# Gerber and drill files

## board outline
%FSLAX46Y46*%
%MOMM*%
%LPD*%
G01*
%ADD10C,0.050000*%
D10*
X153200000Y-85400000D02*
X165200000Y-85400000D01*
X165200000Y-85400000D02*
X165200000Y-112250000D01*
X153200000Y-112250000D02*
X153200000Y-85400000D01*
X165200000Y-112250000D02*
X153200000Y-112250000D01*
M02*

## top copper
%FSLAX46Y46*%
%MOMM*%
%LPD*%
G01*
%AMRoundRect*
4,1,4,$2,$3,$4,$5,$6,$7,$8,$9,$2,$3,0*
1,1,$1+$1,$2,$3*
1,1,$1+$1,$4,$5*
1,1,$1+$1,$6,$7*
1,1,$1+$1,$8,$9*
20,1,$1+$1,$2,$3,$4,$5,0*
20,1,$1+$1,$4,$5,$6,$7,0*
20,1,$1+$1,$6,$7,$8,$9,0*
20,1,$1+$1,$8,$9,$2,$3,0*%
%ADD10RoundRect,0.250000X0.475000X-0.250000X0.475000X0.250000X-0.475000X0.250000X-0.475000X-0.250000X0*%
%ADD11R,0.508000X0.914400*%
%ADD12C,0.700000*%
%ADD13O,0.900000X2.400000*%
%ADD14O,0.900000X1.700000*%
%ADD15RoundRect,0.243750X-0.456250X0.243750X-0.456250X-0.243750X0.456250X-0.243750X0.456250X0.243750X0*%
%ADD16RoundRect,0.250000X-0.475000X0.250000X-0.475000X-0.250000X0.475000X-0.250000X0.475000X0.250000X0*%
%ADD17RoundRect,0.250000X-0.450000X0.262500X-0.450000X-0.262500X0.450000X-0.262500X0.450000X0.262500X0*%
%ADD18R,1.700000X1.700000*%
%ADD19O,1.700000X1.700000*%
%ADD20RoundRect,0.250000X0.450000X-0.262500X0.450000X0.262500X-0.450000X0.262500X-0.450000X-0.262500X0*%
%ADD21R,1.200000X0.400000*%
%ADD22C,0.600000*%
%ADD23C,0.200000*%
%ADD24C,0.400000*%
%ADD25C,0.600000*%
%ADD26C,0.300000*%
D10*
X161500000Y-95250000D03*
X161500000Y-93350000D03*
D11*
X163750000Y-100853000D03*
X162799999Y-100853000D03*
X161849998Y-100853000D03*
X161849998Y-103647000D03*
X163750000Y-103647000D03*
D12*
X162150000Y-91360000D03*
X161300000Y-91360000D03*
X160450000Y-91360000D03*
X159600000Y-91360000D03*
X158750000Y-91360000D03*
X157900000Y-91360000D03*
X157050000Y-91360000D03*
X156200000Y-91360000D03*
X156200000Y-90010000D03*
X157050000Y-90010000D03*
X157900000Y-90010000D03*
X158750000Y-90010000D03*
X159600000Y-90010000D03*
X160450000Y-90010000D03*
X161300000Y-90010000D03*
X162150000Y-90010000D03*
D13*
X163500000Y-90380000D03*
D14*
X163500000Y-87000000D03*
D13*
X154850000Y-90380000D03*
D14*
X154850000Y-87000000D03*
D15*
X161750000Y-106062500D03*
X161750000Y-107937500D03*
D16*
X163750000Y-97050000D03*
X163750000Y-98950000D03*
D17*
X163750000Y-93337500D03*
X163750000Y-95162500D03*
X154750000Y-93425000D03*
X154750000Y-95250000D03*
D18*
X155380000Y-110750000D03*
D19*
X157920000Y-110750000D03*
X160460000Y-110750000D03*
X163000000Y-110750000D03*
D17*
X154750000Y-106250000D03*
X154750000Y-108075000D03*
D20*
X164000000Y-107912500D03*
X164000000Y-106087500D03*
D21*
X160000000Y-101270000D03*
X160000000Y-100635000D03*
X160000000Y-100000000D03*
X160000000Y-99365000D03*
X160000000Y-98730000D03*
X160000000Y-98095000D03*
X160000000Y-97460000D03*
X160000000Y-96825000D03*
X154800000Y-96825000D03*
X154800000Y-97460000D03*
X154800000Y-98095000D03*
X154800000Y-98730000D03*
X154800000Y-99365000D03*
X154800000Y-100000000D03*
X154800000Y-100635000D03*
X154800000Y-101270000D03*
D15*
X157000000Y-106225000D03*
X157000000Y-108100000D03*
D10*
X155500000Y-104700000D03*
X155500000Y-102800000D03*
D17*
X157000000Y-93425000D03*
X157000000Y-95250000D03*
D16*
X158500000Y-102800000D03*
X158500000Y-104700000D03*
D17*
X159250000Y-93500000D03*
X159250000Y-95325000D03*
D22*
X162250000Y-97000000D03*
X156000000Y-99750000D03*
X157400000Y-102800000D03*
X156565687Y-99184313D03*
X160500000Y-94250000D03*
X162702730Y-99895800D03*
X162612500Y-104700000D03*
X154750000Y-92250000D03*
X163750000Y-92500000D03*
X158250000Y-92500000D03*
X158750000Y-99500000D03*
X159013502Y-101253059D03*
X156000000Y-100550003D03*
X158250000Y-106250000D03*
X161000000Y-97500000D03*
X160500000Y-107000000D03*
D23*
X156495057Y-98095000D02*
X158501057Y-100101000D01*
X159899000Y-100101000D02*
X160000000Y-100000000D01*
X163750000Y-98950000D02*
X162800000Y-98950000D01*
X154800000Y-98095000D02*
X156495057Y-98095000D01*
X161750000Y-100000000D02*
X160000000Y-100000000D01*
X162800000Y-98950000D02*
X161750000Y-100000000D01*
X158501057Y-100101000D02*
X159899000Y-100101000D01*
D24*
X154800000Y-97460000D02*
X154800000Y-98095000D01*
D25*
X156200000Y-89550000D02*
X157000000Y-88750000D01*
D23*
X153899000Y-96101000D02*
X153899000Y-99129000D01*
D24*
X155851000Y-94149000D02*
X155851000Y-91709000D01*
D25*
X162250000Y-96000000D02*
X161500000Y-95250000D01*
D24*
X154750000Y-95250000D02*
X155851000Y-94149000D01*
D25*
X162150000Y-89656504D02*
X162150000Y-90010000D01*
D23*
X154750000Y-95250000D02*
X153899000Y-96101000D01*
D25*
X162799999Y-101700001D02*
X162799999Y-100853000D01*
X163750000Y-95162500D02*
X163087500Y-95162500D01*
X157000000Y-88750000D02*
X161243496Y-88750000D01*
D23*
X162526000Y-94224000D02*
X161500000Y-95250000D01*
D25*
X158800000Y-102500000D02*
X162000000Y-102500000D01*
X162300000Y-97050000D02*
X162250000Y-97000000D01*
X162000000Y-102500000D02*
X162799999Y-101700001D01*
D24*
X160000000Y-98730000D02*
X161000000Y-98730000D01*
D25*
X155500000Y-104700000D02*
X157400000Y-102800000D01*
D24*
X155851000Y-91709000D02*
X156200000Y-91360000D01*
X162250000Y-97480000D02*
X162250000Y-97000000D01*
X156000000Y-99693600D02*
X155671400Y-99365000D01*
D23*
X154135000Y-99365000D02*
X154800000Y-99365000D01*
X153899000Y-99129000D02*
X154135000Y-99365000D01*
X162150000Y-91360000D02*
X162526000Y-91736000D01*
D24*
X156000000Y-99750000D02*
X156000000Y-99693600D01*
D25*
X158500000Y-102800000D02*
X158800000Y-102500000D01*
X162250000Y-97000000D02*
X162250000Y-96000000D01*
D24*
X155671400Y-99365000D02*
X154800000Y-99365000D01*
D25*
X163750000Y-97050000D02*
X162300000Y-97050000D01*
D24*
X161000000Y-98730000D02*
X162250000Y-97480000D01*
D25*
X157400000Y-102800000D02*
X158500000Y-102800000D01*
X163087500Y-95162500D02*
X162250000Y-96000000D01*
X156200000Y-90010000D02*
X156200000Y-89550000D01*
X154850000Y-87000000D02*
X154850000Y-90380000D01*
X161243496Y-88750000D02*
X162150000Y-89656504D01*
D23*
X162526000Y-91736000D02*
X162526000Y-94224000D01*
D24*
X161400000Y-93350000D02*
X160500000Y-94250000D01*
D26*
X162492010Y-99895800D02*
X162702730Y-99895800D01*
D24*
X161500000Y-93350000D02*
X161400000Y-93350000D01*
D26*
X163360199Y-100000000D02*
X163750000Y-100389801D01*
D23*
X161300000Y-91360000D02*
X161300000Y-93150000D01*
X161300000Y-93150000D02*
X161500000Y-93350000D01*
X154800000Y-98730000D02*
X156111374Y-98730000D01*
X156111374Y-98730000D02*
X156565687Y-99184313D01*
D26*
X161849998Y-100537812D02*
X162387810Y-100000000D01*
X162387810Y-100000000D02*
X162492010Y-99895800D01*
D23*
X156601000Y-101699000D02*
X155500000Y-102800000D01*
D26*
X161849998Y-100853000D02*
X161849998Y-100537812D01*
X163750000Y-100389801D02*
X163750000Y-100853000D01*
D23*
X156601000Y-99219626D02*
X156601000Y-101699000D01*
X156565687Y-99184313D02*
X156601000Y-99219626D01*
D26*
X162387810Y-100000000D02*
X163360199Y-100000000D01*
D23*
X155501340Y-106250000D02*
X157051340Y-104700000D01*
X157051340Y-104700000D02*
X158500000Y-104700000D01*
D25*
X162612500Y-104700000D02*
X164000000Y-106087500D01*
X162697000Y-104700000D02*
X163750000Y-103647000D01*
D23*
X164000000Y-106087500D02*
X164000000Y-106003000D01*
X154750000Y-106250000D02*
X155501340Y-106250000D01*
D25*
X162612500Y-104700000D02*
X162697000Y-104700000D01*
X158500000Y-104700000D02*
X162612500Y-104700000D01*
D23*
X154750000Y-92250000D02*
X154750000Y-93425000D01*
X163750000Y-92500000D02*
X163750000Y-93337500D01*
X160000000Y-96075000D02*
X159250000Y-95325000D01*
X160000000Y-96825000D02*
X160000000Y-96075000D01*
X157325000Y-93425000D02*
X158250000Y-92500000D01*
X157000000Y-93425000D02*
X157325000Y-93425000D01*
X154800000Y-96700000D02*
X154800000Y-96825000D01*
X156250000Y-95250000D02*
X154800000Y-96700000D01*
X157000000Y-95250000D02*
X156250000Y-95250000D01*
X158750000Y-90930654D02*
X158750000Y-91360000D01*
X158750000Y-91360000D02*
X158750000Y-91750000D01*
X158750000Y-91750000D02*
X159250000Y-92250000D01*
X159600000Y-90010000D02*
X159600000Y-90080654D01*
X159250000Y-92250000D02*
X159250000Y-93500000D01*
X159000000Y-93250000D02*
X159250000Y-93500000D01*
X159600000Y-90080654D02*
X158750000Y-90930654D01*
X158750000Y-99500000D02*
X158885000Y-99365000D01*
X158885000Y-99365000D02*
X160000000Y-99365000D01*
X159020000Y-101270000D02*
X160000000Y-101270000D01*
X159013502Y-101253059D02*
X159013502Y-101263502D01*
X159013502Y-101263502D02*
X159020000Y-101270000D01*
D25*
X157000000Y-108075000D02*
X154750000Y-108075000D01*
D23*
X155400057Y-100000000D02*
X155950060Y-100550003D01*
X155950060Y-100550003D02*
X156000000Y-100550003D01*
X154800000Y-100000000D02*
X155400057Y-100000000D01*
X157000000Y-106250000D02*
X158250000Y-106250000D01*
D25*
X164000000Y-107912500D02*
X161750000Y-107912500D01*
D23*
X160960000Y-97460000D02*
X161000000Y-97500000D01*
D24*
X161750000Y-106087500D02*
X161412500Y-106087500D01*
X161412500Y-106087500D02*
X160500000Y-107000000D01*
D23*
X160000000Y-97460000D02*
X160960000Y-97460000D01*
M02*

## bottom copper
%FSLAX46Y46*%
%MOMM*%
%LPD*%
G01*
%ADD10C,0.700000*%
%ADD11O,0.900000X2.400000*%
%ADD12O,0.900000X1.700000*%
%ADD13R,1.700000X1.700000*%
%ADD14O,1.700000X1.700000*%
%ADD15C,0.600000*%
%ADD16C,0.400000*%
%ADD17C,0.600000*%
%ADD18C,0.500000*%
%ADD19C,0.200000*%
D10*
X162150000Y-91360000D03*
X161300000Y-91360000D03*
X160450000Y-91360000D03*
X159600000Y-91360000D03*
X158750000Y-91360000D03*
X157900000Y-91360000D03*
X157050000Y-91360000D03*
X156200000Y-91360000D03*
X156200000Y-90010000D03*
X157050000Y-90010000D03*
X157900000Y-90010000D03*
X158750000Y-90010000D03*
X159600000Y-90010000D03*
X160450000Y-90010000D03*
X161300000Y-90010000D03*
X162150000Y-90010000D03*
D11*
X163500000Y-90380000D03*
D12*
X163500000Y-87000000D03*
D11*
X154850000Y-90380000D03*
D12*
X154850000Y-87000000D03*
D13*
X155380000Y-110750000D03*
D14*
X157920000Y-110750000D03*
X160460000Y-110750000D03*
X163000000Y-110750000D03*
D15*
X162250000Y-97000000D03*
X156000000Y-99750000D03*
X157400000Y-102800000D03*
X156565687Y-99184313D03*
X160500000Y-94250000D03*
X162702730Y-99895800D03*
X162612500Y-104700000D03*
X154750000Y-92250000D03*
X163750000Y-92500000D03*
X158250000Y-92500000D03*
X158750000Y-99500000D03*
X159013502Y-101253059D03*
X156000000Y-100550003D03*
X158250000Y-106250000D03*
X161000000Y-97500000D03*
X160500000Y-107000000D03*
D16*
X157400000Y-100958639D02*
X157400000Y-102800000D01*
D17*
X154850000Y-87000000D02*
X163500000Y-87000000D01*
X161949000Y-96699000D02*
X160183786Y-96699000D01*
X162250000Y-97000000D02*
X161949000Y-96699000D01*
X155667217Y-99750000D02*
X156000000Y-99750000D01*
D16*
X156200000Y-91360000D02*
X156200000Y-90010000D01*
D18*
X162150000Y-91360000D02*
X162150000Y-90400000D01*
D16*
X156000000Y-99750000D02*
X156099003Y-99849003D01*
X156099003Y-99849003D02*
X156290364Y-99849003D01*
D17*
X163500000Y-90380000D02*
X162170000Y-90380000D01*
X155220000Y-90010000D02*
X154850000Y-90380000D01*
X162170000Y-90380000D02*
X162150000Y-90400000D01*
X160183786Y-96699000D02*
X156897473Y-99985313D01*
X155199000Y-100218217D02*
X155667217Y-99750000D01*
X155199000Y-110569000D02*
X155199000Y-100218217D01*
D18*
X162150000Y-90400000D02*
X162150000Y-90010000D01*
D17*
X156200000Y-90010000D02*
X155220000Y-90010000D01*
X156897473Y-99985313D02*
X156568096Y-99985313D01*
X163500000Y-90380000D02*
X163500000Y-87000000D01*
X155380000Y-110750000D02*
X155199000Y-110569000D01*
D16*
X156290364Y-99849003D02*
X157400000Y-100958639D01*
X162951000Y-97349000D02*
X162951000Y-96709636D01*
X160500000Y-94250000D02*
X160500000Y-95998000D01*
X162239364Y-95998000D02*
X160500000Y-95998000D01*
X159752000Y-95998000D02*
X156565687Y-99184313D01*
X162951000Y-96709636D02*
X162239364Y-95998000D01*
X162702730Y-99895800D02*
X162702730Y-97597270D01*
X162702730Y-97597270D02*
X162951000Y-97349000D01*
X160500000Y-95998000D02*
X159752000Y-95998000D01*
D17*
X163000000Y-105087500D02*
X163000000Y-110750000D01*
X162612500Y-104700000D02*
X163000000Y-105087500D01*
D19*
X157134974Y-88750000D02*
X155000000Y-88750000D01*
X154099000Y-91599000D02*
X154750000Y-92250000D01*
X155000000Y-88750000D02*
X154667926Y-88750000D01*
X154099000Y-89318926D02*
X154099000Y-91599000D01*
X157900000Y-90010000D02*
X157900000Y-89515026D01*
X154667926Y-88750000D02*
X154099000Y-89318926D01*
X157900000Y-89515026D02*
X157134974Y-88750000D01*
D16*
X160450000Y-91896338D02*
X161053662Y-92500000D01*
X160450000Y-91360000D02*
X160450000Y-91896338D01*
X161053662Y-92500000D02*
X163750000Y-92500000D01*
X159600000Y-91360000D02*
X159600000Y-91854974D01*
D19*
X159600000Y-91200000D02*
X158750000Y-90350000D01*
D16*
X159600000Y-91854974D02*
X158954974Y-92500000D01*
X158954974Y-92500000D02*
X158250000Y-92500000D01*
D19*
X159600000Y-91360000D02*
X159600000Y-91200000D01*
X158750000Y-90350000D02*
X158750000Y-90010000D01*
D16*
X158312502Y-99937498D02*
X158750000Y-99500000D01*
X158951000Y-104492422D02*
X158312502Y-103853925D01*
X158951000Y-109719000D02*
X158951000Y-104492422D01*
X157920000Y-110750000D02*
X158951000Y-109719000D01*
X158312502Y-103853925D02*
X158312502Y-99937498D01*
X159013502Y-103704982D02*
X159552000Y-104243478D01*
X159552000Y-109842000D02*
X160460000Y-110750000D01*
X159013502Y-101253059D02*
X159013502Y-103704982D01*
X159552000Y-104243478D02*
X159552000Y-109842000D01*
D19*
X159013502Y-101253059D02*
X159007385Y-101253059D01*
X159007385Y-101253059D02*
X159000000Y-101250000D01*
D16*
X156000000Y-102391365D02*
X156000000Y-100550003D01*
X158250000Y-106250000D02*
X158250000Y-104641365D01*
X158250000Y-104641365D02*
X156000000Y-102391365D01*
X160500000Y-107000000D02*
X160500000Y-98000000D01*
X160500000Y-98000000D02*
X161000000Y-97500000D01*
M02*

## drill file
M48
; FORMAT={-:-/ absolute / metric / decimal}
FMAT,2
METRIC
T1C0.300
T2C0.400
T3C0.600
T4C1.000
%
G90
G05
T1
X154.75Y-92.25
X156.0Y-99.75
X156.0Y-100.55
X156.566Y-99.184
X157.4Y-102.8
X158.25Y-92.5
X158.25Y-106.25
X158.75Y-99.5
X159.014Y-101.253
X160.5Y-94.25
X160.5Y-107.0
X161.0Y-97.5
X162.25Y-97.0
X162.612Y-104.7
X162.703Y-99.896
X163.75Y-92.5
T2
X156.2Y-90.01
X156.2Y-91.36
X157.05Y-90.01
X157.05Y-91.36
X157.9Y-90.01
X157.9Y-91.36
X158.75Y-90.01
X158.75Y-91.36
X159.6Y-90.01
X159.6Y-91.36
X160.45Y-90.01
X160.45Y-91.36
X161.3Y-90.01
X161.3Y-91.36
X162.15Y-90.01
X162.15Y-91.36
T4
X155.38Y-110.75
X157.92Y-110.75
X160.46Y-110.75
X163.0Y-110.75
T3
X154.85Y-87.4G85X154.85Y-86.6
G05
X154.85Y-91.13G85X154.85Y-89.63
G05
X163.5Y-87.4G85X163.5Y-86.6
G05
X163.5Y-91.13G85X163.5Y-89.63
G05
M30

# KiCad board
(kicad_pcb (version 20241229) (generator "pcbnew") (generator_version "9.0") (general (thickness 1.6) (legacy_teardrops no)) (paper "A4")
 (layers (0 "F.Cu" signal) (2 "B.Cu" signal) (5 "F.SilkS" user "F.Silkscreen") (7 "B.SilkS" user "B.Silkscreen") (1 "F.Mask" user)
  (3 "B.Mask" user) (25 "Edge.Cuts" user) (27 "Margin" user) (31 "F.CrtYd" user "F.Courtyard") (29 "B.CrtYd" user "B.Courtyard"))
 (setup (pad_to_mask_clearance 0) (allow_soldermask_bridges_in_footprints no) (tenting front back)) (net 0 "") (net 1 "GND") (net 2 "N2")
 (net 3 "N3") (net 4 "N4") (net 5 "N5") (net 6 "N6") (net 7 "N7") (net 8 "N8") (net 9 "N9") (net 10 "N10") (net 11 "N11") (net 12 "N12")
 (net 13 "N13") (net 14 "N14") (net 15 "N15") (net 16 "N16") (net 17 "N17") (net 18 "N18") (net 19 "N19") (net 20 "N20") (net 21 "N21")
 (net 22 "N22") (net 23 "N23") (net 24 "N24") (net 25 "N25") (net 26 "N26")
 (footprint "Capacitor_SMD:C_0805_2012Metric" (layer "F.Cu") (at 161.5 94.3 90)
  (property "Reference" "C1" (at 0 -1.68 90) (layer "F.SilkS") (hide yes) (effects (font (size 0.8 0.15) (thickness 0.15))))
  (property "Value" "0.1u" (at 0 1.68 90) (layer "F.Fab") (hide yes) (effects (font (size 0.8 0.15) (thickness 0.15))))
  (pad "1" smd roundrect (at -0.95 0 90) (size 1 1.45) (layers "F.Cu" "F.Mask" "F.Paste") (roundrect_rratio 0.25) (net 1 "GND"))
  (pad "2" smd roundrect (at 0.95 0 90) (size 1 1.45) (layers "F.Cu" "F.Mask" "F.Paste") (roundrect_rratio 0.25) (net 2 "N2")))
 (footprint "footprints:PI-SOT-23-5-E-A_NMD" (layer "F.Cu") (at 162.799999 102.25 -90)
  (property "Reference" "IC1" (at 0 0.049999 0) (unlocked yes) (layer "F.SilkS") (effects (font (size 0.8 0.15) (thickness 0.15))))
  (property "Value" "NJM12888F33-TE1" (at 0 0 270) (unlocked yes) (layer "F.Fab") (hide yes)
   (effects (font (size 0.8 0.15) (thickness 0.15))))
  (pad "1" smd rect (at -1.397 -0.950001 270) (size 0.9144 0.508) (layers "F.Cu" "F.Mask" "F.Paste") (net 2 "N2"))
  (pad "2" smd rect (at -1.397 0 270) (size 0.9144 0.508) (layers "F.Cu" "F.Mask" "F.Paste") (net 1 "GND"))
  (pad "3" smd rect (at -1.397 0.950001 270) (size 0.9144 0.508) (layers "F.Cu" "F.Mask" "F.Paste") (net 2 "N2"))
  (pad "4" smd rect (at 1.397 0.950001 270) (size 0.9144 0.508) (layers "F.Cu" "F.Mask" "F.Paste") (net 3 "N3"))
  (pad "5" smd rect (at 1.397 -0.950001 270) (size 0.9144 0.508) (layers "F.Cu" "F.Mask" "F.Paste") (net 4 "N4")))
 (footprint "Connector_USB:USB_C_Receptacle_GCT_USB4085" (layer "F.Cu") (at 162.15 91.36 180)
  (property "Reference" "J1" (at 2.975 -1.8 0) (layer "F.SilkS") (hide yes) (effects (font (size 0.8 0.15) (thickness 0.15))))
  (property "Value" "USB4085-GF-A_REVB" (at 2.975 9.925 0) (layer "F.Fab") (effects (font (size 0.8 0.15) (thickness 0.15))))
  (pad "A1" thru_hole circle (at 0 0 180) (size 0.7 0.7) (drill 0.4) (layers "*.Cu" "*.Mask") (remove_unused_layers no) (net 1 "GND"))
  (pad "A4" thru_hole circle (at 0.85 0 180) (size 0.7 0.7) (drill 0.4) (layers "*.Cu" "*.Mask") (remove_unused_layers no) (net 2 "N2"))
  (pad "A5" thru_hole circle (at 1.7 0 180) (size 0.7 0.7) (drill 0.4) (layers "*.Cu" "*.Mask") (remove_unused_layers no) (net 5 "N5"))
  (pad "A6" thru_hole circle (at 2.55 0 180) (size 0.7 0.7) (drill 0.4) (layers "*.Cu" "*.Mask") (remove_unused_layers no) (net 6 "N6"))
  (pad "A7" thru_hole circle (at 3.4 0 180) (size 0.7 0.7) (drill 0.4) (layers "*.Cu" "*.Mask") (remove_unused_layers no) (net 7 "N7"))
  (pad "A8" thru_hole circle (at 4.25 0 180) (size 0.7 0.7) (drill 0.4) (layers "*.Cu" "*.Mask") (remove_unused_layers no) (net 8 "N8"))
  (pad "A9" thru_hole circle (at 5.1 0 180) (size 0.7 0.7) (drill 0.4) (layers "*.Cu" "*.Mask") (remove_unused_layers no) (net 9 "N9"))
  (pad "A12" thru_hole circle (at 5.95 0 180) (size 0.7 0.7) (drill 0.4) (layers "*.Cu" "*.Mask") (remove_unused_layers no) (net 1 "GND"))
  (pad "B1" thru_hole circle (at 5.95 1.35 180) (size 0.7 0.7) (drill 0.4) (layers "*.Cu" "*.Mask") (remove_unused_layers no) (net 1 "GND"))
  (pad "B4" thru_hole circle (at 5.1 1.35 180) (size 0.7 0.7) (drill 0.4) (layers "*.Cu" "*.Mask") (remove_unused_layers no) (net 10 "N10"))
  (pad "B5" thru_hole circle (at 4.25 1.35 180) (size 0.7 0.7) (drill 0.4) (layers "*.Cu" "*.Mask") (remove_unused_layers no) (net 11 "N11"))
  (pad "B6" thru_hole circle (at 3.4 1.35 180) (size 0.7 0.7) (drill 0.4) (layers "*.Cu" "*.Mask") (remove_unused_layers no) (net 6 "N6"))
  (pad "B7" thru_hole circle (at 2.55 1.35 180) (size 0.7 0.7) (drill 0.4) (layers "*.Cu" "*.Mask") (remove_unused_layers no) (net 7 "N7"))
  (pad "B8" thru_hole circle (at 1.7 1.35 180) (size 0.7 0.7) (drill 0.4) (layers "*.Cu" "*.Mask") (remove_unused_layers no) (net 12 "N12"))
  (pad "B9" thru_hole circle (at 0.85 1.35 180) (size 0.7 0.7) (drill 0.4) (layers "*.Cu" "*.Mask") (remove_unused_layers no) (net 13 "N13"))
  (pad "B12" thru_hole circle (at 0 1.35 180) (size 0.7 0.7) (drill 0.4) (layers "*.Cu" "*.Mask") (remove_unused_layers no) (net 1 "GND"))
  (pad "S1" thru_hole oval (at -1.35 0.98 180) (size 0.9 2.4) (drill oval 0.6 2.1) (layers "*.Cu" "*.Mask") (remove_unused_layers no)
   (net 1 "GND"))
  (pad "S1" thru_hole oval (at -1.35 4.36 180) (size 0.9 1.7) (drill oval 0.6 1.4) (layers "*.Cu" "*.Mask") (remove_unused_layers no)
   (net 1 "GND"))
  (pad "S1" thru_hole oval (at 7.3 0.98 180) (size 0.9 2.4) (drill oval 0.6 2.1) (layers "*.Cu" "*.Mask") (remove_unused_layers no)
   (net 1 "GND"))
  (pad "S1" thru_hole oval (at 7.3 4.36 180) (size 0.9 1.7) (drill oval 0.6 1.4) (layers "*.Cu" "*.Mask") (remove_unused_layers no)
   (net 1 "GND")))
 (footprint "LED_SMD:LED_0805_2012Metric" (layer "F.Cu") (at 161.75 107 -90)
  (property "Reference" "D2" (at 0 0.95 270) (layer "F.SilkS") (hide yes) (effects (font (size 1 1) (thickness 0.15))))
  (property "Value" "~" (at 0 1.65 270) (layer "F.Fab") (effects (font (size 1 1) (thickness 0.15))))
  (pad "1" smd roundrect (at -0.9375 0 270) (size 0.975 1.4) (layers "F.Cu" "F.Mask" "F.Paste") (roundrect_rratio 0.25) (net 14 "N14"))
  (pad "2" smd roundrect (at 0.9375 0 270) (size 0.975 1.4) (layers "F.Cu" "F.Mask" "F.Paste") (roundrect_rratio 0.25) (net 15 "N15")))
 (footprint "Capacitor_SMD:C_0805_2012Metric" (layer "F.Cu") (at 163.75 98 -90)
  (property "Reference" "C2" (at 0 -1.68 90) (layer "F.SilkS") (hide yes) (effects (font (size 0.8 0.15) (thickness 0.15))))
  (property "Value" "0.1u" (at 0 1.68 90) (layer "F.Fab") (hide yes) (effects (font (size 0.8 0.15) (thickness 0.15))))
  (pad "1" smd roundrect (at -0.95 0 270) (size 1 1.45) (layers "F.Cu" "F.Mask" "F.Paste") (roundrect_rratio 0.25) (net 1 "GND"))
  (pad "2" smd roundrect (at 0.95 0 270) (size 1 1.45) (layers "F.Cu" "F.Mask" "F.Paste") (roundrect_rratio 0.25) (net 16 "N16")))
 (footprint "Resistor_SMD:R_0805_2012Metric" (layer "F.Cu") (at 163.75 94.25 -90)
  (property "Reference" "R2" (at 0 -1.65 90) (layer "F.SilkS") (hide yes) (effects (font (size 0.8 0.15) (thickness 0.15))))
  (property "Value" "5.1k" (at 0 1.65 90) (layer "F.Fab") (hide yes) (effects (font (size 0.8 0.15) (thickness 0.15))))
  (pad "1" smd roundrect (at -0.9125 0 270) (size 1.025 1.4) (layers "F.Cu" "F.Mask" "F.Paste") (roundrect_rratio 0.243902) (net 5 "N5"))
  (pad "2" smd roundrect (at 0.9125 0 270) (size 1.025 1.4) (layers "F.Cu" "F.Mask" "F.Paste") (roundrect_rratio 0.243902) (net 1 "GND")))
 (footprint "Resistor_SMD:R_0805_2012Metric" (layer "F.Cu") (at 154.75 94.3375 -90)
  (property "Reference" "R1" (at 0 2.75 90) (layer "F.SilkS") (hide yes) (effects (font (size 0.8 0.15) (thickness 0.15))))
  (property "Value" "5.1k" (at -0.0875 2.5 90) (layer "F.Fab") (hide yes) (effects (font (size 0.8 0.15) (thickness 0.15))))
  (pad "1" smd roundrect (at -0.9125 0 270) (size 1.025 1.4) (layers "F.Cu" "F.Mask" "F.Paste") (roundrect_rratio 0.243902) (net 11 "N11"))
  (pad "2" smd roundrect (at 0.9125 0 270) (size 1.025 1.4) (layers "F.Cu" "F.Mask" "F.Paste") (roundrect_rratio 0.243902) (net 1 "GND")))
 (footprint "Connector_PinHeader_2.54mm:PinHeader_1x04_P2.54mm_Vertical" (layer "F.Cu") (at 155.38 110.75 90)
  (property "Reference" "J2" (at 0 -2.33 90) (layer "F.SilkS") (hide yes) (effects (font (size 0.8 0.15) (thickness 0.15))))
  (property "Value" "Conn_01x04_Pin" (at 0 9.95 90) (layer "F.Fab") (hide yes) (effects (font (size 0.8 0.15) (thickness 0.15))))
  (pad "1" thru_hole rect (at 0 0 90) (size 1.7 1.7) (drill 1) (layers "*.Cu" "*.Mask") (remove_unused_layers no) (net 1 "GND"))
  (pad "2" thru_hole oval (at 0 2.54 90) (size 1.7 1.7) (drill 1) (layers "*.Cu" "*.Mask") (remove_unused_layers no) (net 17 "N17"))
  (pad "3" thru_hole oval (at 0 5.08 90) (size 1.7 1.7) (drill 1) (layers "*.Cu" "*.Mask") (remove_unused_layers no) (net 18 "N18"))
  (pad "4" thru_hole oval (at 0 7.62 90) (size 1.7 1.7) (drill 1) (layers "*.Cu" "*.Mask") (remove_unused_layers no) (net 4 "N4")))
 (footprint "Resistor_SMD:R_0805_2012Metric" (layer "F.Cu") (at 154.75 107.1625 -90)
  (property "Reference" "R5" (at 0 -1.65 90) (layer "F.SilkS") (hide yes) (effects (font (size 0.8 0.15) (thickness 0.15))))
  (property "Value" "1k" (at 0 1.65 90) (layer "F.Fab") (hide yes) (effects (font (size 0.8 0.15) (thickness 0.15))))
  (pad "1" smd roundrect (at -0.9125 0 270) (size 1.025 1.4) (layers "F.Cu" "F.Mask" "F.Paste") (roundrect_rratio 0.243902) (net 4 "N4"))
  (pad "2" smd roundrect (at 0.9125 0 270) (size 1.025 1.4) (layers "F.Cu" "F.Mask" "F.Paste") (roundrect_rratio 0.243902) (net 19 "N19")))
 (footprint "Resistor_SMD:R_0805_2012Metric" (layer "F.Cu") (at 164 107 90)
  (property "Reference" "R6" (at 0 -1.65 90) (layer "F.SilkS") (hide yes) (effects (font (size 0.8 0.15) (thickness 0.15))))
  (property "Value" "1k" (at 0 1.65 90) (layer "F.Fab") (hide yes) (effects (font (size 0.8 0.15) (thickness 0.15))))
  (pad "1" smd roundrect (at -0.9125 0 90) (size 1.025 1.4) (layers "F.Cu" "F.Mask" "F.Paste") (roundrect_rratio 0.243902) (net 15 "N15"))
  (pad "2" smd roundrect (at 0.9125 0 90) (size 1.025 1.4) (layers "F.Cu" "F.Mask" "F.Paste") (roundrect_rratio 0.243902) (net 4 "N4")))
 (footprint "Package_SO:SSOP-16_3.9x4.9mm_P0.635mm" (layer "F.Cu") (at 157.4 99.0475 180)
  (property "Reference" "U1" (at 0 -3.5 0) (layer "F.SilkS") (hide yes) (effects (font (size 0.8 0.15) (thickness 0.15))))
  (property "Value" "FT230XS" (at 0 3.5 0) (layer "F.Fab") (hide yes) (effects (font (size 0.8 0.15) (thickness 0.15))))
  (pad "1" smd rect (at -2.6 -2.2225 180) (size 1.2 0.4) (layers "F.Cu" "F.Mask" "F.Paste") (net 18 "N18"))
  (pad "2" smd rect (at -2.6 -1.5875 180) (size 1.2 0.4) (layers "F.Cu" "F.Mask" "F.Paste") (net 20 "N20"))
  (pad "3" smd rect (at -2.6 -0.9525 180) (size 1.2 0.4) (layers "F.Cu" "F.Mask" "F.Paste") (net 16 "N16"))
  (pad "4" smd rect (at -2.6 -0.3175 180) (size 1.2 0.4) (layers "F.Cu" "F.Mask" "F.Paste") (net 17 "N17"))
  (pad "5" smd rect (at -2.6 0.3175 180) (size 1.2 0.4) (layers "F.Cu" "F.Mask" "F.Paste") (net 1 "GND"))
  (pad "6" smd rect (at -2.6 0.9525 180) (size 1.2 0.4) (layers "F.Cu" "F.Mask" "F.Paste") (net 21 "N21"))
  (pad "7" smd rect (at -2.6 1.5875 180) (size 1.2 0.4) (layers "F.Cu" "F.Mask" "F.Paste") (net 14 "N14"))
  (pad "8" smd rect (at -2.6 2.2225 180) (size 1.2 0.4) (layers "F.Cu" "F.Mask" "F.Paste") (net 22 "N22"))
  (pad "9" smd rect (at 2.6 2.2225 180) (size 1.2 0.4) (layers "F.Cu" "F.Mask" "F.Paste") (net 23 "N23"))
  (pad "10" smd rect (at 2.6 1.5875 180) (size 1.2 0.4) (layers "F.Cu" "F.Mask" "F.Paste") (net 16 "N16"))
  (pad "11" smd rect (at 2.6 0.9525 180) (size 1.2 0.4) (layers "F.Cu" "F.Mask" "F.Paste") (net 16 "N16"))
  (pad "12" smd rect (at 2.6 0.3175 180) (size 1.2 0.4) (layers "F.Cu" "F.Mask" "F.Paste") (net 2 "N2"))
  (pad "13" smd rect (at 2.6 -0.3175 180) (size 1.2 0.4) (layers "F.Cu" "F.Mask" "F.Paste") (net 1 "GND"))
  (pad "14" smd rect (at 2.6 -0.9525 180) (size 1.2 0.4) (layers "F.Cu" "F.Mask" "F.Paste") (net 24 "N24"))
  (pad "15" smd rect (at 2.6 -1.5875 180) (size 1.2 0.4) (layers "F.Cu" "F.Mask" "F.Paste") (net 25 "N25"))
  (pad "16" smd rect (at 2.6 -2.2225 180) (size 1.2 0.4) (layers "F.Cu" "F.Mask" "F.Paste") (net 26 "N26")))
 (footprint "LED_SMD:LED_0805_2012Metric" (layer "F.Cu") (at 157 107.1625 -90)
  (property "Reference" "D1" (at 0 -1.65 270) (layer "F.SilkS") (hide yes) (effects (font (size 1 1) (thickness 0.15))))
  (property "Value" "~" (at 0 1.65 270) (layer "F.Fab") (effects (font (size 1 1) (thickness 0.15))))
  (pad "1" smd roundrect (at -0.9375 0 270) (size 0.975 1.4) (layers "F.Cu" "F.Mask" "F.Paste") (roundrect_rratio 0.25) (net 24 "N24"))
  (pad "2" smd roundrect (at 0.9375 0 270) (size 0.975 1.4) (layers "F.Cu" "F.Mask" "F.Paste") (roundrect_rratio 0.25) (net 19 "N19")))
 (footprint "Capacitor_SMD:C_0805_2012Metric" (layer "F.Cu") (at 155.5 103.75 90)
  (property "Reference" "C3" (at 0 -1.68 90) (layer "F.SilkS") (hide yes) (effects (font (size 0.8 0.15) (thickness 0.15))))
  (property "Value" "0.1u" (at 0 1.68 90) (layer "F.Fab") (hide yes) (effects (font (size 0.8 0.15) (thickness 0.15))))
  (pad "1" smd roundrect (at -0.95 0 90) (size 1 1.45) (layers "F.Cu" "F.Mask" "F.Paste") (roundrect_rratio 0.25) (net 1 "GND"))
  (pad "2" smd roundrect (at 0.95 0 90) (size 1 1.45) (layers "F.Cu" "F.Mask" "F.Paste") (roundrect_rratio 0.25) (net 2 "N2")))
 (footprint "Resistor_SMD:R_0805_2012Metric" (layer "F.Cu") (at 157 94.3375 -90)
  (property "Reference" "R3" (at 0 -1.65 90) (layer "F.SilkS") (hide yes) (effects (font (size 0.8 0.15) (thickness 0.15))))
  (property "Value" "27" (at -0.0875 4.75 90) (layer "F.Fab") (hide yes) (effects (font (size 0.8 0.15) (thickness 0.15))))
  (pad "1" smd roundrect (at -0.9125 0 270) (size 1.025 1.4) (layers "F.Cu" "F.Mask" "F.Paste") (roundrect_rratio 0.243902) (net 6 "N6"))
  (pad "2" smd roundrect (at 0.9125 0 270) (size 1.025 1.4) (layers "F.Cu" "F.Mask" "F.Paste") (roundrect_rratio 0.243902) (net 23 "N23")))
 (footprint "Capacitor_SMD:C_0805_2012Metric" (layer "F.Cu") (at 158.5 103.75 -90)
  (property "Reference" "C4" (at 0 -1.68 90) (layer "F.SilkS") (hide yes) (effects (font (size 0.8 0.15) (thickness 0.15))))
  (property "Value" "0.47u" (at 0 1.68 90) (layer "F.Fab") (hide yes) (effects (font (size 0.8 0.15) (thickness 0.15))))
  (pad "1" smd roundrect (at -0.95 0 270) (size 1 1.45) (layers "F.Cu" "F.Mask" "F.Paste") (roundrect_rratio 0.25) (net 1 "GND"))
  (pad "2" smd roundrect (at 0.95 0 270) (size 1 1.45) (layers "F.Cu" "F.Mask" "F.Paste") (roundrect_rratio 0.25) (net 4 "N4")))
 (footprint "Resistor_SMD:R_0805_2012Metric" (layer "F.Cu") (at 159.25 94.4125 -90)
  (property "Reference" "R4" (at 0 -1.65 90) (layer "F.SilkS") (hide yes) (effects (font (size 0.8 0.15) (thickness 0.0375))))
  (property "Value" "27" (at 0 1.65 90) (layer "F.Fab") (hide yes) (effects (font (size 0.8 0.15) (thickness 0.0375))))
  (pad "1" smd roundrect (at -0.9125 0 270) (size 1.025 1.4) (layers "F.Cu" "F.Mask" "F.Paste") (roundrect_rratio 0.243902) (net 7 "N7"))
  (pad "2" smd roundrect (at 0.9125 0 270) (size 1.025 1.4) (layers "F.Cu" "F.Mask" "F.Paste") (roundrect_rratio 0.243902) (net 22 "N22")))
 (gr_line (start 153.2 85.4) (end 165.2 85.4) (stroke (width 0.05) (type default)) (layer "Edge.Cuts"))
 (gr_line (start 165.2 85.4) (end 165.2 112.25) (stroke (width 0.05) (type default)) (layer "Edge.Cuts"))
 (gr_line (start 153.2 112.25) (end 153.2 85.4) (stroke (width 0.05) (type default)) (layer "Edge.Cuts"))
 (gr_line (start 165.2 112.25) (end 153.2 112.25) (stroke (width 0.05) (type default)) (layer "Edge.Cuts"))
 (segment (start 156.495057 98.095) (end 158.501057 100.101) (width 0.2) (layer "F.Cu") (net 16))
 (segment (start 159.899 100.101) (end 160 100) (width 0.2) (layer "F.Cu") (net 16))
 (segment (start 163.75 98.95) (end 162.8 98.95) (width 0.2) (layer "F.Cu") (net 16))
 (segment (start 154.8 98.095) (end 156.495057 98.095) (width 0.2) (layer "F.Cu") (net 16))
 (segment (start 161.75 100) (end 160 100) (width 0.2) (layer "F.Cu") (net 16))
 (segment (start 162.8 98.95) (end 161.75 100) (width 0.2) (layer "F.Cu") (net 16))
 (segment (start 158.501057 100.101) (end 159.899 100.101) (width 0.2) (layer "F.Cu") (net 16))
 (segment (start 154.8 97.46) (end 154.8 98.095) (width 0.4) (layer "F.Cu") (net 16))
 (segment (start 156.2 89.55) (end 157 88.75) (width 0.6) (layer "F.Cu") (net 1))
 (segment (start 153.899 96.101) (end 153.899 99.129) (width 0.2) (layer "F.Cu") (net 1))
 (segment (start 155.851 94.149) (end 155.851 91.709) (width 0.4) (layer "F.Cu") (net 1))
 (segment (start 162.25 96) (end 161.5 95.25) (width 0.6) (layer "F.Cu") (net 1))
 (segment (start 154.75 95.25) (end 155.851 94.149) (width 0.4) (layer "F.Cu") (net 1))
 (segment (start 162.15 89.656504) (end 162.15 90.01) (width 0.6) (layer "F.Cu") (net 1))
 (segment (start 154.75 95.25) (end 153.899 96.101) (width 0.2) (layer "F.Cu") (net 1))
 (segment (start 162.799999 101.700001) (end 162.799999 100.853) (width 0.6) (layer "F.Cu") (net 1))
 (segment (start 163.75 95.1625) (end 163.0875 95.1625) (width 0.6) (layer "F.Cu") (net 1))
 (segment (start 157 88.75) (end 161.243496 88.75) (width 0.6) (layer "F.Cu") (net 1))
 (segment (start 162.526 94.224) (end 161.5 95.25) (width 0.2) (layer "F.Cu") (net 1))
 (segment (start 158.8 102.5) (end 162 102.5) (width 0.6) (layer "F.Cu") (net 1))
 (segment (start 162.3 97.05) (end 162.25 97) (width 0.6) (layer "F.Cu") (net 1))
 (segment (start 162 102.5) (end 162.799999 101.700001) (width 0.6) (layer "F.Cu") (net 1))
 (segment (start 160 98.73) (end 161 98.73) (width 0.4) (layer "F.Cu") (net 1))
 (segment (start 155.5 104.7) (end 157.4 102.8) (width 0.6) (layer "F.Cu") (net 1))
 (segment (start 155.851 91.709) (end 156.2 91.36) (width 0.4) (layer "F.Cu") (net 1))
 (segment (start 162.25 97.48) (end 162.25 97) (width 0.4) (layer "F.Cu") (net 1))
 (segment (start 156 99.6936) (end 155.6714 99.365) (width 0.4) (layer "F.Cu") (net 1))
 (segment (start 154.135 99.365) (end 154.8 99.365) (width 0.2) (layer "F.Cu") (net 1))
 (segment (start 153.899 99.129) (end 154.135 99.365) (width 0.2) (layer "F.Cu") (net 1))
 (segment (start 162.15 91.36) (end 162.526 91.736) (width 0.2) (layer "F.Cu") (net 1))
 (segment (start 156 99.75) (end 156 99.6936) (width 0.4) (layer "F.Cu") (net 1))
 (segment (start 158.5 102.8) (end 158.8 102.5) (width 0.6) (layer "F.Cu") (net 1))
 (segment (start 162.25 97) (end 162.25 96) (width 0.6) (layer "F.Cu") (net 1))
 (segment (start 155.6714 99.365) (end 154.8 99.365) (width 0.4) (layer "F.Cu") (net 1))
 (segment (start 163.75 97.05) (end 162.3 97.05) (width 0.6) (layer "F.Cu") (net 1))
 (segment (start 161 98.73) (end 162.25 97.48) (width 0.4) (layer "F.Cu") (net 1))
 (segment (start 157.4 102.8) (end 158.5 102.8) (width 0.6) (layer "F.Cu") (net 1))
 (segment (start 163.0875 95.1625) (end 162.25 96) (width 0.6) (layer "F.Cu") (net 1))
 (segment (start 156.2 90.01) (end 156.2 89.55) (width 0.6) (layer "F.Cu") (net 1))
 (segment (start 154.85 87) (end 154.85 90.38) (width 0.6) (layer "F.Cu") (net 1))
 (segment (start 161.243496 88.75) (end 162.15 89.656504) (width 0.6) (layer "F.Cu") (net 1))
 (segment (start 162.526 91.736) (end 162.526 94.224) (width 0.2) (layer "F.Cu") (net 1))
 (via (at 162.25 97) (size 0.6) (drill 0.3) (layers "F.Cu" "B.Cu") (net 1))
 (via (at 156 99.75) (size 0.6) (drill 0.3) (layers "F.Cu" "B.Cu") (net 1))
 (via (at 157.4 102.8) (size 0.6) (drill 0.3) (layers "F.Cu" "B.Cu") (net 1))
 (segment (start 157.4 100.958639) (end 157.4 102.8) (width 0.4) (layer "B.Cu") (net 1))
 (segment (start 154.85 87) (end 163.5 87) (width 0.6) (layer "B.Cu") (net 1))
 (segment (start 161.949 96.699) (end 160.183786 96.699) (width 0.6) (layer "B.Cu") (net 1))
 (segment (start 162.25 97) (end 161.949 96.699) (width 0.6) (layer "B.Cu") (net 1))
 (segment (start 155.667217 99.75) (end 156 99.75) (width 0.6) (layer "B.Cu") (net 1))
 (segment (start 156.2 91.36) (end 156.2 90.01) (width 0.4) (layer "B.Cu") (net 1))
 (segment (start 162.15 91.36) (end 162.15 90.4) (width 0.5) (layer "B.Cu") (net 1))
 (segment (start 156 99.75) (end 156.099003 99.849003) (width 0.4) (layer "B.Cu") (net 1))
 (segment (start 156.099003 99.849003) (end 156.290364 99.849003) (width 0.4) (layer "B.Cu") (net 1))
 (segment (start 163.5 90.38) (end 162.17 90.38) (width 0.6) (layer "B.Cu") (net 1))
 (segment (start 155.22 90.01) (end 154.85 90.38) (width 0.6) (layer "B.Cu") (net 1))
 (segment (start 162.17 90.38) (end 162.15 90.4) (width 0.6) (layer "B.Cu") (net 1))
 (segment (start 160.183786 96.699) (end 156.897473 99.985313) (width 0.6) (layer "B.Cu") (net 1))
 (segment (start 155.199 100.218217) (end 155.667217 99.75) (width 0.6) (layer "B.Cu") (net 1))
 (segment (start 155.199 110.569) (end 155.199 100.218217) (width 0.6) (layer "B.Cu") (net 1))
 (segment (start 162.15 90.4) (end 162.15 90.01) (width 0.5) (layer "B.Cu") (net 1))
 (segment (start 156.2 90.01) (end 155.22 90.01) (width 0.6) (layer "B.Cu") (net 1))
 (segment (start 156.897473 99.985313) (end 156.568096 99.985313) (width 0.6) (layer "B.Cu") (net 1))
 (segment (start 163.5 90.38) (end 163.5 87) (width 0.6) (layer "B.Cu") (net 1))
 (segment (start 155.38 110.75) (end 155.199 110.569) (width 0.6) (layer "B.Cu") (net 1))
 (segment (start 156.290364 99.849003) (end 157.4 100.958639) (width 0.4) (layer "B.Cu") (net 1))
 (segment (start 161.4 93.35) (end 160.5 94.25) (width 0.4) (layer "F.Cu") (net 2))
 (segment (start 162.49201 99.8958) (end 162.70273 99.8958) (width 0.3) (layer "F.Cu") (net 2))
 (segment (start 161.5 93.35) (end 161.4 93.35) (width 0.4) (layer "F.Cu") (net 2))
 (segment (start 163.360199 100) (end 163.75 100.389801) (width 0.3) (layer "F.Cu") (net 2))
 (segment (start 161.3 91.36) (end 161.3 93.15) (width 0.2) (layer "F.Cu") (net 2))
 (segment (start 161.3 93.15) (end 161.5 93.35) (width 0.2) (layer "F.Cu") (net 2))
 (segment (start 154.8 98.73) (end 156.111374 98.73) (width 0.2) (layer "F.Cu") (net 2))
 (segment (start 156.111374 98.73) (end 156.565687 99.184313) (width 0.2) (layer "F.Cu") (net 2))
 (segment (start 161.849998 100.537812) (end 162.38781 100) (width 0.3) (layer "F.Cu") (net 2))
 (segment (start 162.38781 100) (end 162.49201 99.8958) (width 0.3) (layer "F.Cu") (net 2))
 (segment (start 156.601 101.699) (end 155.5 102.8) (width 0.2) (layer "F.Cu") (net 2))
 (segment (start 161.849998 100.853) (end 161.849998 100.537812) (width 0.3) (layer "F.Cu") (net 2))
 (segment (start 163.75 100.389801) (end 163.75 100.853) (width 0.3) (layer "F.Cu") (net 2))
 (segment (start 156.601 99.219626) (end 156.601 101.699) (width 0.2) (layer "F.Cu") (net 2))
 (segment (start 156.565687 99.184313) (end 156.601 99.219626) (width 0.2) (layer "F.Cu") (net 2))
 (segment (start 162.38781 100) (end 163.360199 100) (width 0.3) (layer "F.Cu") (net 2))
 (via (at 156.565687 99.184313) (size 0.6) (drill 0.3) (layers "F.Cu" "B.Cu") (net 2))
 (via (at 160.5 94.25) (size 0.6) (drill 0.3) (layers "F.Cu" "B.Cu") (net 2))
 (via (at 162.70273 99.8958) (size 0.6) (drill 0.3) (layers "F.Cu" "B.Cu") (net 2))
 (segment (start 162.951 97.349) (end 162.951 96.709636) (width 0.4) (layer "B.Cu") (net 2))
 (segment (start 160.5 94.25) (end 160.5 95.998) (width 0.4) (layer "B.Cu") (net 2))
 (segment (start 162.239364 95.998) (end 160.5 95.998) (width 0.4) (layer "B.Cu") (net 2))
 (segment (start 159.752 95.998) (end 156.565687 99.184313) (width 0.4) (layer "B.Cu") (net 2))
 (segment (start 162.951 96.709636) (end 162.239364 95.998) (width 0.4) (layer "B.Cu") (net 2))
 (segment (start 162.70273 99.8958) (end 162.70273 97.59727) (width 0.4) (layer "B.Cu") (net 2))
 (segment (start 162.70273 97.59727) (end 162.951 97.349) (width 0.4) (layer "B.Cu") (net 2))
 (segment (start 160.5 95.998) (end 159.752 95.998) (width 0.4) (layer "B.Cu") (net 2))
 (segment (start 155.50134 106.25) (end 157.05134 104.7) (width 0.2) (layer "F.Cu") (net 4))
 (segment (start 157.05134 104.7) (end 158.5 104.7) (width 0.2) (layer "F.Cu") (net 4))
 (segment (start 162.6125 104.7) (end 164 106.0875) (width 0.6) (layer "F.Cu") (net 4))
 (segment (start 162.697 104.7) (end 163.75 103.647) (width 0.6) (layer "F.Cu") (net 4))
 (segment (start 164 106.0875) (end 164 106.003) (width 0.2) (layer "F.Cu") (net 4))
 (segment (start 154.75 106.25) (end 155.50134 106.25) (width 0.2) (layer "F.Cu") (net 4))
 (segment (start 162.6125 104.7) (end 162.697 104.7) (width 0.6) (layer "F.Cu") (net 4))
 (segment (start 158.5 104.7) (end 162.6125 104.7) (width 0.6) (layer "F.Cu") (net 4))
 (via (at 162.6125 104.7) (size 0.6) (drill 0.3) (layers "F.Cu" "B.Cu") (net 4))
 (segment (start 163 105.0875) (end 163 110.75) (width 0.6) (layer "B.Cu") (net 4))
 (segment (start 162.6125 104.7) (end 163 105.0875) (width 0.6) (layer "B.Cu") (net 4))
 (segment (start 154.75 92.25) (end 154.75 93.425) (width 0.2) (layer "F.Cu") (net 11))
 (via (at 154.75 92.25) (size 0.6) (drill 0.3) (layers "F.Cu" "B.Cu") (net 11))
 (segment (start 157.134974 88.75) (end 155 88.75) (width 0.2) (layer "B.Cu") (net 11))
 (segment (start 154.099 91.599) (end 154.75 92.25) (width 0.2) (layer "B.Cu") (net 11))
 (segment (start 155 88.75) (end 154.667926 88.75) (width 0.2) (layer "B.Cu") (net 11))
 (segment (start 154.099 89.318926) (end 154.099 91.599) (width 0.2) (layer "B.Cu") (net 11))
 (segment (start 157.9 90.01) (end 157.9 89.515026) (width 0.2) (layer "B.Cu") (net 11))
 (segment (start 154.667926 88.75) (end 154.099 89.318926) (width 0.2) (layer "B.Cu") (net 11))
 (segment (start 157.9 89.515026) (end 157.134974 88.75) (width 0.2) (layer "B.Cu") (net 11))
 (segment (start 163.75 92.5) (end 163.75 93.3375) (width 0.2) (layer "F.Cu") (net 5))
 (via (at 163.75 92.5) (size 0.6) (drill 0.3) (layers "F.Cu" "B.Cu") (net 5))
 (segment (start 160.45 91.896338) (end 161.053662 92.5) (width 0.4) (layer "B.Cu") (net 5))
 (segment (start 160.45 91.36) (end 160.45 91.896338) (width 0.4) (layer "B.Cu") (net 5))
 (segment (start 161.053662 92.5) (end 163.75 92.5) (width 0.4) (layer "B.Cu") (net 5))
 (segment (start 160 96.075) (end 159.25 95.325) (width 0.2) (layer "F.Cu") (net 22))
 (segment (start 160 96.825) (end 160 96.075) (width 0.2) (layer "F.Cu") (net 22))
 (segment (start 157.325 93.425) (end 158.25 92.5) (width 0.2) (layer "F.Cu") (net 6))
 (segment (start 157 93.425) (end 157.325 93.425) (width 0.2) (layer "F.Cu") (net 6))
 (via (at 158.25 92.5) (size 0.6) (drill 0.3) (layers "F.Cu" "B.Cu") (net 6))
 (segment (start 159.6 91.36) (end 159.6 91.854974) (width 0.4) (layer "B.Cu") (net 6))
 (segment (start 159.6 91.2) (end 158.75 90.35) (width 0.2) (layer "B.Cu") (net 6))
 (segment (start 159.6 91.854974) (end 158.954974 92.5) (width 0.4) (layer "B.Cu") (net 6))
 (segment (start 158.954974 92.5) (end 158.25 92.5) (width 0.4) (layer "B.Cu") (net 6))
 (segment (start 159.6 91.36) (end 159.6 91.2) (width 0.2) (layer "B.Cu") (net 6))
 (segment (start 158.75 90.35) (end 158.75 90.01) (width 0.2) (layer "B.Cu") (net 6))
 (segment (start 154.8 96.7) (end 154.8 96.825) (width 0.2) (layer "F.Cu") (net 23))
 (segment (start 156.25 95.25) (end 154.8 96.7) (width 0.2) (layer "F.Cu") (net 23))
 (segment (start 157 95.25) (end 156.25 95.25) (width 0.2) (layer "F.Cu") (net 23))
 (segment (start 158.75 90.930654) (end 158.75 91.36) (width 0.2) (layer "F.Cu") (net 7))
 (segment (start 158.75 91.36) (end 158.75 91.75) (width 0.2) (layer "F.Cu") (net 7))
 (segment (start 158.75 91.75) (end 159.25 92.25) (width 0.2) (layer "F.Cu") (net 7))
 (segment (start 159.6 90.01) (end 159.6 90.080654) (width 0.2) (layer "F.Cu") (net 7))
 (segment (start 159.25 92.25) (end 159.25 93.5) (width 0.2) (layer "F.Cu") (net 7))
 (segment (start 159 93.25) (end 159.25 93.5) (width 0.2) (layer "F.Cu") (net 7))
 (segment (start 159.6 90.080654) (end 158.75 90.930654) (width 0.2) (layer "F.Cu") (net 7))
 (segment (start 158.75 99.5) (end 158.885 99.365) (width 0.2) (layer "F.Cu") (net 17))
 (segment (start 158.885 99.365) (end 160 99.365) (width 0.2) (layer "F.Cu") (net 17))
 (via (at 158.75 99.5) (size 0.6) (drill 0.3) (layers "F.Cu" "B.Cu") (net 17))
 (segment (start 158.312502 99.937498) (end 158.75 99.5) (width 0.4) (layer "B.Cu") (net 17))
 (segment (start 158.951 104.492422) (end 158.312502 103.853925) (width 0.4) (layer "B.Cu") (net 17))
 (segment (start 158.951 109.719) (end 158.951 104.492422) (width 0.4) (layer "B.Cu") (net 17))
 (segment (start 157.92 110.75) (end 158.951 109.719) (width 0.4) (layer "B.Cu") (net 17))
 (segment (start 158.312502 103.853925) (end 158.312502 99.937498) (width 0.4) (layer "B.Cu") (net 17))
 (segment (start 159.02 101.27) (end 160 101.27) (width 0.2) (layer "F.Cu") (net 18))
 (segment (start 159.013502 101.253059) (end 159.013502 101.263502) (width 0.2) (layer "F.Cu") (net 18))
 (segment (start 159.013502 101.263502) (end 159.02 101.27) (width 0.2) (layer "F.Cu") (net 18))
 (via (at 159.013502 101.253059) (size 0.6) (drill 0.3) (layers "F.Cu" "B.Cu") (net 18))
 (segment (start 159.013502 103.704982) (end 159.552 104.243478) (width 0.4) (layer "B.Cu") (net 18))
 (segment (start 159.552 109.842) (end 160.46 110.75) (width 0.4) (layer "B.Cu") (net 18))
 (segment (start 159.013502 101.253059) (end 159.013502 103.704982) (width 0.4) (layer "B.Cu") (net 18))
 (segment (start 159.552 104.243478) (end 159.552 109.842) (width 0.4) (layer "B.Cu") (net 18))
 (segment (start 159.013502 101.253059) (end 159.007385 101.253059) (width 0.2) (layer "B.Cu") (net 18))
 (segment (start 159.007385 101.253059) (end 159 101.25) (width 0.2) (layer "B.Cu") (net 18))
 (segment (start 157 108.075) (end 154.75 108.075) (width 0.6) (layer "F.Cu") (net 19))
 (segment (start 155.400057 100) (end 155.95006 100.550003) (width 0.2) (layer "F.Cu") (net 24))
 (segment (start 155.95006 100.550003) (end 156 100.550003) (width 0.2) (layer "F.Cu") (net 24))
 (segment (start 154.8 100) (end 155.400057 100) (width 0.2) (layer "F.Cu") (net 24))
 (segment (start 157 106.25) (end 158.25 106.25) (width 0.2) (layer "F.Cu") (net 24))
 (via (at 156 100.550003) (size 0.6) (drill 0.3) (layers "F.Cu" "B.Cu") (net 24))
 (via (at 158.25 106.25) (size 0.6) (drill 0.3) (layers "F.Cu" "B.Cu") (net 24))
 (segment (start 156 102.391365) (end 156 100.550003) (width 0.4) (layer "B.Cu") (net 24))
 (segment (start 158.25 106.25) (end 158.25 104.641365) (width 0.4) (layer "B.Cu") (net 24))
 (segment (start 158.25 104.641365) (end 156 102.391365) (width 0.4) (layer "B.Cu") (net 24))
 (segment (start 164 107.9125) (end 161.75 107.9125) (width 0.6) (layer "F.Cu") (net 15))
 (segment (start 160.96 97.46) (end 161 97.5) (width 0.2) (layer "F.Cu") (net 14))
 (segment (start 161.75 106.0875) (end 161.4125 106.0875) (width 0.4) (layer "F.Cu") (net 14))
 (segment (start 161.4125 106.0875) (end 160.5 107) (width 0.4) (layer "F.Cu") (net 14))
 (segment (start 160 97.46) (end 160.96 97.46) (width 0.2) (layer "F.Cu") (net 14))
 (via (at 161 97.5) (size 0.6) (drill 0.3) (layers "F.Cu" "B.Cu") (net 14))
 (via (at 160.5 107) (size 0.6) (drill 0.3) (layers "F.Cu" "B.Cu") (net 14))
 (segment (start 160.5 107) (end 160.5 98) (width 0.4) (layer "B.Cu") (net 14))
 (segment (start 160.5 98) (end 161 97.5) (width 0.4) (layer "B.Cu") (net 14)))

